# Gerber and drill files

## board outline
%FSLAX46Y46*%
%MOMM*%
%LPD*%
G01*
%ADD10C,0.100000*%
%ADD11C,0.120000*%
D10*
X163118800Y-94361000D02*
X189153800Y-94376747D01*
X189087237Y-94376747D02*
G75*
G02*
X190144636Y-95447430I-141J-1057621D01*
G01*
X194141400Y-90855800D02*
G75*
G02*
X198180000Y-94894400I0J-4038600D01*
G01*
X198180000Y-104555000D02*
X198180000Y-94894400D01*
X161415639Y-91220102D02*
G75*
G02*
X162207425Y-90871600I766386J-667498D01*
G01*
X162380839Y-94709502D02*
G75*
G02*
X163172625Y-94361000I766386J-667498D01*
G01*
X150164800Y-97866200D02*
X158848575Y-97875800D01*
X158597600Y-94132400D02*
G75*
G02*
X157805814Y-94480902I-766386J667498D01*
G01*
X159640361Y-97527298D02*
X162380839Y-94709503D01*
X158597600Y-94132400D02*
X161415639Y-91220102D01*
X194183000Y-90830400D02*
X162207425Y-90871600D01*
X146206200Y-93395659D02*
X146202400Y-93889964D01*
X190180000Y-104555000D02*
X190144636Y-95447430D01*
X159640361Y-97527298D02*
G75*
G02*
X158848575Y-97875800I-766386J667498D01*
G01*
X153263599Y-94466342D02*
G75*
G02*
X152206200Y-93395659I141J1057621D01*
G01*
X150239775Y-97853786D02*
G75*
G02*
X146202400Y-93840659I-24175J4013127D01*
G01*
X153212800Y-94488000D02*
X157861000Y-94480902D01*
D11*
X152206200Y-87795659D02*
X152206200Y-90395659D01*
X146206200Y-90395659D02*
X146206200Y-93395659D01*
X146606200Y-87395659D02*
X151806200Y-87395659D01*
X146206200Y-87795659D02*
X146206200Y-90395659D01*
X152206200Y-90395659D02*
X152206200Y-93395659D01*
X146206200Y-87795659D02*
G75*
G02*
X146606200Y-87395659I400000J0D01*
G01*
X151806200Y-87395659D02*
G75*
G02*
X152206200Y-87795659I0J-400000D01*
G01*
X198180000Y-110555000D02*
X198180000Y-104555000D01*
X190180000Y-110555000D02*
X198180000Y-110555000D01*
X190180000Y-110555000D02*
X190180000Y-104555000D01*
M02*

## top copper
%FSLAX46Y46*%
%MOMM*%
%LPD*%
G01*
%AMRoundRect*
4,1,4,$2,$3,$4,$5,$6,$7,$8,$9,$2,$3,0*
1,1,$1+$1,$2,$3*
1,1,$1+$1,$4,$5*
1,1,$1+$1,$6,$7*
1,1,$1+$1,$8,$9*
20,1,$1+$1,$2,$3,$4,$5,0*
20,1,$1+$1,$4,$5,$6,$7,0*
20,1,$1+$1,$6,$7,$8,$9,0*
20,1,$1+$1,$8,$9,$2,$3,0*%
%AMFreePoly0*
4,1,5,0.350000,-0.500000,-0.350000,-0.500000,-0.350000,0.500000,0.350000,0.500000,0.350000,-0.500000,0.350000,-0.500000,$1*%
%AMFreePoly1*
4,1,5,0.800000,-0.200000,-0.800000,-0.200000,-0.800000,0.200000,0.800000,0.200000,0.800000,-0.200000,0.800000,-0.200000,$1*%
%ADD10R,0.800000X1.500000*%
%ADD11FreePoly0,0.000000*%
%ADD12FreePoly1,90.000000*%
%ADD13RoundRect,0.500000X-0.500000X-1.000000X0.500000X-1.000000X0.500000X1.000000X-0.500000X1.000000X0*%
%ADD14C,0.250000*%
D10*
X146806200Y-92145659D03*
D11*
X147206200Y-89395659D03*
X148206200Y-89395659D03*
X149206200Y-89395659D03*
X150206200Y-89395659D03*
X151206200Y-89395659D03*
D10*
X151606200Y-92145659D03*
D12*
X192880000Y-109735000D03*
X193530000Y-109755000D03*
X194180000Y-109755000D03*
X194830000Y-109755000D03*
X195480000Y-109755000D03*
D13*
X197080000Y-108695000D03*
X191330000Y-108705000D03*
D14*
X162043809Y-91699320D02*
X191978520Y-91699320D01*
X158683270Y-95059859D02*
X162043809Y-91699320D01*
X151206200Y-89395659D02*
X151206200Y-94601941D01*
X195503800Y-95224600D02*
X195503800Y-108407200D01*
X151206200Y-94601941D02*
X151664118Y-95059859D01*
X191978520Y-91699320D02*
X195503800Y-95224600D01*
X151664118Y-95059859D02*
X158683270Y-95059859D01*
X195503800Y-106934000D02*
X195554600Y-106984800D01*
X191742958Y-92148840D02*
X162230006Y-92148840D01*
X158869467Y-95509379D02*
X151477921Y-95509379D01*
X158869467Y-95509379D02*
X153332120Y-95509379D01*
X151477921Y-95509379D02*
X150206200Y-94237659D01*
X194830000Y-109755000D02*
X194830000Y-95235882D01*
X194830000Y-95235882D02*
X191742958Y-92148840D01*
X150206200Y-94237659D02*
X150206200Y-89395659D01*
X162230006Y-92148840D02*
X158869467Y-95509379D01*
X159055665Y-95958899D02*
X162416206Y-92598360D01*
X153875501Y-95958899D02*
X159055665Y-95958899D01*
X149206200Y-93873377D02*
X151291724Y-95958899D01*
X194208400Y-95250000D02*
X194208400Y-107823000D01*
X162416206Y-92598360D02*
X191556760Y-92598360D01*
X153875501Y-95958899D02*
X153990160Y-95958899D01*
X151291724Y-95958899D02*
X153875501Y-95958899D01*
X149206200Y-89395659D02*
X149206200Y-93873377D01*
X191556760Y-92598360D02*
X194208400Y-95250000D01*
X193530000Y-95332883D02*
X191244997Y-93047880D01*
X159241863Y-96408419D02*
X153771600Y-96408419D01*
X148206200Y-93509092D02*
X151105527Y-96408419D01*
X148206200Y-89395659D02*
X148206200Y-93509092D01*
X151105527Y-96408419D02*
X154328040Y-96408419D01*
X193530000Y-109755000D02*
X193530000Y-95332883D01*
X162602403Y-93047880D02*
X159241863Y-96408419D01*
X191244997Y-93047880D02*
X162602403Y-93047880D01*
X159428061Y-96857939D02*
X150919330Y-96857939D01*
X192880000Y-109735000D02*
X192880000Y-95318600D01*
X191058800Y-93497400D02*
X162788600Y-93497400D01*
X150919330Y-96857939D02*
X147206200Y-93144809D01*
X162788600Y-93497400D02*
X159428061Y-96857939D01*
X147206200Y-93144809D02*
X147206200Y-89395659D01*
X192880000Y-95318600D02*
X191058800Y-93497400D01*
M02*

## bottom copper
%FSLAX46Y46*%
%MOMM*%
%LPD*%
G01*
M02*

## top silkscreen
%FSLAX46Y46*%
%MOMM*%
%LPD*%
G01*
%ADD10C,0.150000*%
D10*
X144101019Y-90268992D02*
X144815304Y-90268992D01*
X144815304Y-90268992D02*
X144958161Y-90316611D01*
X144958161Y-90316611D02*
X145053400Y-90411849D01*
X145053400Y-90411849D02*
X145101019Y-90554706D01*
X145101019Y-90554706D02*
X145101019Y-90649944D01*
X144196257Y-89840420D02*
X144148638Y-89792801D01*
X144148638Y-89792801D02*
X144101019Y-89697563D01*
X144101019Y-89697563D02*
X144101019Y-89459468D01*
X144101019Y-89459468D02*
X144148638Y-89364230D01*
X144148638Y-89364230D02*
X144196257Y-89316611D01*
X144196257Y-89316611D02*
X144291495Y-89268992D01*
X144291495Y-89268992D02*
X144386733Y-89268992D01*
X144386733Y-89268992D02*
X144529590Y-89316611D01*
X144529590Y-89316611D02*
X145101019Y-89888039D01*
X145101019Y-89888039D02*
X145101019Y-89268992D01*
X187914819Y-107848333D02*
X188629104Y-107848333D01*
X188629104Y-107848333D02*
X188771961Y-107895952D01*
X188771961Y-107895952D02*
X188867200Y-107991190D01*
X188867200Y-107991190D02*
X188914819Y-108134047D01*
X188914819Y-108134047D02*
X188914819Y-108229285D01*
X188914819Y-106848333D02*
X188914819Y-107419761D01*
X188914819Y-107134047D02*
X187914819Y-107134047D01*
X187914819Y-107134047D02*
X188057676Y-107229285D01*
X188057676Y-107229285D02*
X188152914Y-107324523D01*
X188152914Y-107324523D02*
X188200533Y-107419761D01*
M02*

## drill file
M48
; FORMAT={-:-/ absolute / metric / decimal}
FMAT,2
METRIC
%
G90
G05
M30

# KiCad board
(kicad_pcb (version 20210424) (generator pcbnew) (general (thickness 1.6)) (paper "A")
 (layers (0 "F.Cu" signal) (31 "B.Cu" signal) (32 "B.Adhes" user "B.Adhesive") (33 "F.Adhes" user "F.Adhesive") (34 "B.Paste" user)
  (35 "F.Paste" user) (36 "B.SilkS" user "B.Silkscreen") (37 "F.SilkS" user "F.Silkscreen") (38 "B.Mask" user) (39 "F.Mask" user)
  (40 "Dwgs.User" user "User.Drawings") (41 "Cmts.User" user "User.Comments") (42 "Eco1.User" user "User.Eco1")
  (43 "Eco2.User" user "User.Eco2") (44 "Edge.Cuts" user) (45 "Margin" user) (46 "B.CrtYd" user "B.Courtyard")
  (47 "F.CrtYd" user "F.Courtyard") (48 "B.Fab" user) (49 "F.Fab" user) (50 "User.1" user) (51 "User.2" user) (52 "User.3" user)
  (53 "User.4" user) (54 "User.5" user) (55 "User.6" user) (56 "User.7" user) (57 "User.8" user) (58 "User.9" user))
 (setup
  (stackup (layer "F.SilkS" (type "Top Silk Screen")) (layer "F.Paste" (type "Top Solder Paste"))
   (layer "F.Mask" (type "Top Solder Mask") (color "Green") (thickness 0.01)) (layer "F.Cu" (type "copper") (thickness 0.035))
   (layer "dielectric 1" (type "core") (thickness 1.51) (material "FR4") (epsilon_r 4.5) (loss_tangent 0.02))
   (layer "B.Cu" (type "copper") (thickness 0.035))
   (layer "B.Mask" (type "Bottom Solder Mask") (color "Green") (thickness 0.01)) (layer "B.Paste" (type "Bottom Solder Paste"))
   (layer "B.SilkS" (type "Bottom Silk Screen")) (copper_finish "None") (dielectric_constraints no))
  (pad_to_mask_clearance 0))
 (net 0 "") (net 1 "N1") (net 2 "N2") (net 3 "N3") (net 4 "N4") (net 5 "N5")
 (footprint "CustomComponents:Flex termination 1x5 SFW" (layer "F.Cu") (at 149.2062 90.395659)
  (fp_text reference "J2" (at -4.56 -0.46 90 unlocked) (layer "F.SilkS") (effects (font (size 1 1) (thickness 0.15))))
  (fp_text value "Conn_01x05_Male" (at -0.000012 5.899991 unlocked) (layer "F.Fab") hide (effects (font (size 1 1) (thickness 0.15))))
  (fp_line (start 3 -2.6) (end 3 0) (layer "Edge.Cuts") (width 0.12))
  (fp_line (start -3 0) (end -3 3) (layer "Edge.Cuts") (width 0.12))
  (fp_line (start -2.6 -3) (end 2.6 -3) (layer "Edge.Cuts") (width 0.12))
  (fp_line (start -3 -2.6) (end -3 0) (layer "Edge.Cuts") (width 0.12))
  (fp_line (start 3 0) (end 3 3) (layer "Edge.Cuts") (width 0.12))
  (fp_arc (start -2.6 -2.6) (end -2.6 -3) (angle -90) (layer "Edge.Cuts") (width 0.12))
  (fp_arc (start 2.6 -2.6) (end 2.6 -3) (angle 90) (layer "Edge.Cuts") (width 0.12))
  (pad "1" connect rect (at -2.4 1.75) (size 0.8 1.5) (layers "F.Cu" "F.Mask") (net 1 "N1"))
  (pad "1" connect custom (at -2 -1) (size 0.7 1) (layers "F.Cu" "F.Mask") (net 1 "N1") (options (clearance outline) (anchor rect))
   (primitives))
  (pad "2" connect custom (at -1 -1) (size 0.7 1) (layers "F.Cu" "F.Mask") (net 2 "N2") (options (clearance outline) (anchor rect))
   (primitives))
  (pad "3" connect custom (at 0 -1) (size 0.7 1) (layers "F.Cu" "F.Mask") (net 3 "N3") (options (clearance outline) (anchor rect))
   (primitives))
  (pad "4" connect custom (at 1 -1) (size 0.7 1) (layers "F.Cu" "F.Mask") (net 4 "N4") (options (clearance outline) (anchor rect))
   (primitives))
  (pad "5" connect custom (at 2 -1) (size 0.7 1) (layers "F.Cu" "F.Mask") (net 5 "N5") (options (clearance outline) (anchor rect))
   (primitives))
  (pad "5" connect rect (at 2.4 1.75) (size 0.8 1.5) (layers "F.Cu" "F.Mask") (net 5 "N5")))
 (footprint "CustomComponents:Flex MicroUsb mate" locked (layer "F.Cu") (at 194.18 112.555)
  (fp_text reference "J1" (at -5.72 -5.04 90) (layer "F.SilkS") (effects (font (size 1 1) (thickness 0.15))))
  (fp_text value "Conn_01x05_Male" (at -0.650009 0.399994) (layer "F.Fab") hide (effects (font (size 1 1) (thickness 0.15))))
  (fp_line (start 4 -2) (end 4 -8) (layer "Edge.Cuts") (width 0.12))
  (fp_line (start -4 -2) (end 4 -2) (layer "Edge.Cuts") (width 0.12))
  (fp_line (start -4 -2) (end -4 -8) (layer "Edge.Cuts") (width 0.12))
  (pad "1" smd custom locked (at -1.3 -2.82 90) (size 1.6 0.4) (layers "F.Cu" "F.Paste" "F.Mask") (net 1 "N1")
   (options (clearance outline) (anchor rect)) (primitives))
  (pad "2" smd custom locked (at -0.65 -2.8 90) (size 1.6 0.4) (layers "F.Cu" "F.Paste" "F.Mask") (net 2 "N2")
   (options (clearance outline) (anchor rect)) (primitives))
  (pad "3" smd custom locked (at 0 -2.8 90) (size 1.6 0.4) (layers "F.Cu" "F.Paste" "F.Mask") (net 3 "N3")
   (options (clearance outline) (anchor rect)) (primitives))
  (pad "4" smd custom locked (at 0.65 -2.8 90) (size 1.6 0.4) (layers "F.Cu" "F.Paste" "F.Mask") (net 4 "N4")
   (options (clearance outline) (anchor rect)) (primitives))
  (pad "5" smd custom locked (at 1.3 -2.8 90) (size 1.6 0.4) (layers "F.Cu" "F.Paste" "F.Mask") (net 5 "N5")
   (options (clearance outline) (anchor rect)) (primitives))
  (pad "6" smd roundrect locked (at 2.9 -3.86) (size 2 3) (layers "F.Cu" "F.Paste" "F.Mask") (roundrect_rratio 0.25))
  (pad "6" smd roundrect locked (at -2.85 -3.85) (size 2 3) (layers "F.Cu" "F.Paste" "F.Mask") (roundrect_rratio 0.25)))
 (gr_line (start 163.1188 94.361) (end 189.1538 94.376747) (layer "Edge.Cuts") (width 0.1))
 (gr_arc (start 189.087096 95.434368) (end 190.144636 95.44743) (angle -90.7) (layer "Edge.Cuts") (width 0.1))
 (gr_arc (start 194.1414 94.8944) (end 198.18 94.8944) (angle -90) (layer "Edge.Cuts") (width 0.1))
 (gr_line (start 198.18 104.555) (end 198.18 94.8944) (layer "Edge.Cuts") (width 0.1))
 (gr_arc (start 162.182025 91.8876) (end 162.207425 90.8716) (angle -50.37728241) (layer "Edge.Cuts") (width 0.1))
 (gr_arc (start 163.147225 95.377) (end 163.172625 94.361) (angle -50.37728241) (layer "Edge.Cuts") (width 0.1))
 (gr_line (start 150.1648 97.8662) (end 158.848575 97.8758) (layer "Edge.Cuts") (width 0.1))
 (gr_arc (start 157.831214 93.464902) (end 157.805814 94.480902) (angle -50.37728241) (layer "Edge.Cuts") (width 0.1))
 (gr_line (start 159.640361 97.527298) (end 162.380839 94.709503) (layer "Edge.Cuts") (width 0.1))
 (gr_line (start 158.5976 94.1324) (end 161.415639 91.220102) (layer "Edge.Cuts") (width 0.1))
 (gr_line (start 194.183 90.8304) (end 162.207425 90.8716) (layer "Edge.Cuts") (width 0.1))
 (gr_line (start 146.2062 93.395659) (end 146.2024 93.889964) (layer "Edge.Cuts") (width 0.1))
 (gr_line (start 190.18 104.555) (end 190.144636 95.44743) (layer "Edge.Cuts") (width 0.1))
 (gr_arc (start 158.873975 96.8598) (end 158.848575 97.8758) (angle -50.37728241) (layer "Edge.Cuts") (width 0.1))
 (gr_arc (start 153.26374 93.408721) (end 152.2062 93.395659) (angle -90.7) (layer "Edge.Cuts") (width 0.1))
 (gr_arc (start 150.2156 93.840659) (end 146.2024 93.840659) (angle -90.34515112) (layer "Edge.Cuts") (width 0.1))
 (gr_line (start 153.2128 94.488) (end 157.861 94.480902) (layer "Edge.Cuts") (width 0.1))
 (segment (start 162.043809 91.69932) (end 191.97852 91.69932) (width 0.25) (layer "F.Cu") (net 5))
 (segment (start 158.68327 95.059859) (end 162.043809 91.69932) (width 0.25) (layer "F.Cu") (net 5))
 (segment (start 151.2062 89.395659) (end 151.2062 94.601941) (width 0.25) (layer "F.Cu") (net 5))
 (segment (start 195.5038 95.2246) (end 195.5038 108.4072) (width 0.25) (layer "F.Cu") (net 5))
 (segment (start 151.2062 94.601941) (end 151.664118 95.059859) (width 0.25) (layer "F.Cu") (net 5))
 (segment (start 191.97852 91.69932) (end 195.5038 95.2246) (width 0.25) (layer "F.Cu") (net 5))
 (segment (start 151.664118 95.059859) (end 158.68327 95.059859) (width 0.25) (layer "F.Cu") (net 5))
 (segment (start 195.5038 106.934) (end 195.5546 106.9848) (width 0.25) (layer "F.Cu") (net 5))
 (segment (start 191.742958 92.14884) (end 162.230006 92.14884) (width 0.25) (layer "F.Cu") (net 4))
 (segment (start 158.869467 95.509379) (end 151.477921 95.509379) (width 0.25) (layer "F.Cu") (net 4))
 (segment (start 158.869467 95.509379) (end 153.33212 95.509379) (width 0.25) (layer "F.Cu") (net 4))
 (segment (start 151.477921 95.509379) (end 150.2062 94.237659) (width 0.25) (layer "F.Cu") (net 4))
 (segment (start 194.83 109.755) (end 194.83 95.235882) (width 0.25) (layer "F.Cu") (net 4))
 (segment (start 194.83 95.235882) (end 191.742958 92.14884) (width 0.25) (layer "F.Cu") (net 4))
 (segment (start 150.2062 94.237659) (end 150.2062 89.395659) (width 0.25) (layer "F.Cu") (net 4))
 (segment (start 162.230006 92.14884) (end 158.869467 95.509379) (width 0.25) (layer "F.Cu") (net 4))
 (segment (start 159.055665 95.958899) (end 162.416206 92.59836) (width 0.25) (layer "F.Cu") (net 3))
 (segment (start 153.875501 95.958899) (end 159.055665 95.958899) (width 0.25) (layer "F.Cu") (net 3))
 (segment (start 149.2062 93.873377) (end 151.291724 95.958899) (width 0.25) (layer "F.Cu") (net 3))
 (segment (start 194.2084 95.25) (end 194.2084 107.823) (width 0.25) (layer "F.Cu") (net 3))
 (segment (start 162.416206 92.59836) (end 191.55676 92.59836) (width 0.25) (layer "F.Cu") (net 3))
 (segment (start 153.875501 95.958899) (end 153.99016 95.958899) (width 0.25) (layer "F.Cu") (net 3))
 (segment (start 151.291724 95.958899) (end 153.875501 95.958899) (width 0.25) (layer "F.Cu") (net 3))
 (segment (start 149.2062 89.395659) (end 149.2062 93.873377) (width 0.25) (layer "F.Cu") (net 3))
 (segment (start 191.55676 92.59836) (end 194.2084 95.25) (width 0.25) (layer "F.Cu") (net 3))
 (segment (start 193.53 95.332883) (end 191.244997 93.04788) (width 0.25) (layer "F.Cu") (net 2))
 (segment (start 159.241863 96.408419) (end 153.7716 96.408419) (width 0.25) (layer "F.Cu") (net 2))
 (segment (start 148.2062 93.509092) (end 151.105527 96.408419) (width 0.25) (layer "F.Cu") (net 2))
 (segment (start 148.2062 89.395659) (end 148.2062 93.509092) (width 0.25) (layer "F.Cu") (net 2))
 (segment (start 151.105527 96.408419) (end 154.32804 96.408419) (width 0.25) (layer "F.Cu") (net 2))
 (segment (start 193.53 109.755) (end 193.53 95.332883) (width 0.25) (layer "F.Cu") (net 2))
 (segment (start 162.602403 93.04788) (end 159.241863 96.408419) (width 0.25) (layer "F.Cu") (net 2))
 (segment (start 191.244997 93.04788) (end 162.602403 93.04788) (width 0.25) (layer "F.Cu") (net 2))
 (segment (start 159.428061 96.857939) (end 150.91933 96.857939) (width 0.25) (layer "F.Cu") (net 1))
 (segment (start 192.88 109.735) (end 192.88 95.3186) (width 0.25) (layer "F.Cu") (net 1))
 (segment (start 191.0588 93.4974) (end 162.7886 93.4974) (width 0.25) (layer "F.Cu") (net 1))
 (segment (start 150.91933 96.857939) (end 147.2062 93.144809) (width 0.25) (layer "F.Cu") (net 1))
 (segment (start 162.7886 93.4974) (end 159.428061 96.857939) (width 0.25) (layer "F.Cu") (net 1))
 (segment (start 147.2062 93.144809) (end 147.2062 89.395659) (width 0.25) (layer "F.Cu") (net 1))
 (segment (start 192.88 95.3186) (end 191.0588 93.4974) (width 0.25) (layer "F.Cu") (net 1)))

